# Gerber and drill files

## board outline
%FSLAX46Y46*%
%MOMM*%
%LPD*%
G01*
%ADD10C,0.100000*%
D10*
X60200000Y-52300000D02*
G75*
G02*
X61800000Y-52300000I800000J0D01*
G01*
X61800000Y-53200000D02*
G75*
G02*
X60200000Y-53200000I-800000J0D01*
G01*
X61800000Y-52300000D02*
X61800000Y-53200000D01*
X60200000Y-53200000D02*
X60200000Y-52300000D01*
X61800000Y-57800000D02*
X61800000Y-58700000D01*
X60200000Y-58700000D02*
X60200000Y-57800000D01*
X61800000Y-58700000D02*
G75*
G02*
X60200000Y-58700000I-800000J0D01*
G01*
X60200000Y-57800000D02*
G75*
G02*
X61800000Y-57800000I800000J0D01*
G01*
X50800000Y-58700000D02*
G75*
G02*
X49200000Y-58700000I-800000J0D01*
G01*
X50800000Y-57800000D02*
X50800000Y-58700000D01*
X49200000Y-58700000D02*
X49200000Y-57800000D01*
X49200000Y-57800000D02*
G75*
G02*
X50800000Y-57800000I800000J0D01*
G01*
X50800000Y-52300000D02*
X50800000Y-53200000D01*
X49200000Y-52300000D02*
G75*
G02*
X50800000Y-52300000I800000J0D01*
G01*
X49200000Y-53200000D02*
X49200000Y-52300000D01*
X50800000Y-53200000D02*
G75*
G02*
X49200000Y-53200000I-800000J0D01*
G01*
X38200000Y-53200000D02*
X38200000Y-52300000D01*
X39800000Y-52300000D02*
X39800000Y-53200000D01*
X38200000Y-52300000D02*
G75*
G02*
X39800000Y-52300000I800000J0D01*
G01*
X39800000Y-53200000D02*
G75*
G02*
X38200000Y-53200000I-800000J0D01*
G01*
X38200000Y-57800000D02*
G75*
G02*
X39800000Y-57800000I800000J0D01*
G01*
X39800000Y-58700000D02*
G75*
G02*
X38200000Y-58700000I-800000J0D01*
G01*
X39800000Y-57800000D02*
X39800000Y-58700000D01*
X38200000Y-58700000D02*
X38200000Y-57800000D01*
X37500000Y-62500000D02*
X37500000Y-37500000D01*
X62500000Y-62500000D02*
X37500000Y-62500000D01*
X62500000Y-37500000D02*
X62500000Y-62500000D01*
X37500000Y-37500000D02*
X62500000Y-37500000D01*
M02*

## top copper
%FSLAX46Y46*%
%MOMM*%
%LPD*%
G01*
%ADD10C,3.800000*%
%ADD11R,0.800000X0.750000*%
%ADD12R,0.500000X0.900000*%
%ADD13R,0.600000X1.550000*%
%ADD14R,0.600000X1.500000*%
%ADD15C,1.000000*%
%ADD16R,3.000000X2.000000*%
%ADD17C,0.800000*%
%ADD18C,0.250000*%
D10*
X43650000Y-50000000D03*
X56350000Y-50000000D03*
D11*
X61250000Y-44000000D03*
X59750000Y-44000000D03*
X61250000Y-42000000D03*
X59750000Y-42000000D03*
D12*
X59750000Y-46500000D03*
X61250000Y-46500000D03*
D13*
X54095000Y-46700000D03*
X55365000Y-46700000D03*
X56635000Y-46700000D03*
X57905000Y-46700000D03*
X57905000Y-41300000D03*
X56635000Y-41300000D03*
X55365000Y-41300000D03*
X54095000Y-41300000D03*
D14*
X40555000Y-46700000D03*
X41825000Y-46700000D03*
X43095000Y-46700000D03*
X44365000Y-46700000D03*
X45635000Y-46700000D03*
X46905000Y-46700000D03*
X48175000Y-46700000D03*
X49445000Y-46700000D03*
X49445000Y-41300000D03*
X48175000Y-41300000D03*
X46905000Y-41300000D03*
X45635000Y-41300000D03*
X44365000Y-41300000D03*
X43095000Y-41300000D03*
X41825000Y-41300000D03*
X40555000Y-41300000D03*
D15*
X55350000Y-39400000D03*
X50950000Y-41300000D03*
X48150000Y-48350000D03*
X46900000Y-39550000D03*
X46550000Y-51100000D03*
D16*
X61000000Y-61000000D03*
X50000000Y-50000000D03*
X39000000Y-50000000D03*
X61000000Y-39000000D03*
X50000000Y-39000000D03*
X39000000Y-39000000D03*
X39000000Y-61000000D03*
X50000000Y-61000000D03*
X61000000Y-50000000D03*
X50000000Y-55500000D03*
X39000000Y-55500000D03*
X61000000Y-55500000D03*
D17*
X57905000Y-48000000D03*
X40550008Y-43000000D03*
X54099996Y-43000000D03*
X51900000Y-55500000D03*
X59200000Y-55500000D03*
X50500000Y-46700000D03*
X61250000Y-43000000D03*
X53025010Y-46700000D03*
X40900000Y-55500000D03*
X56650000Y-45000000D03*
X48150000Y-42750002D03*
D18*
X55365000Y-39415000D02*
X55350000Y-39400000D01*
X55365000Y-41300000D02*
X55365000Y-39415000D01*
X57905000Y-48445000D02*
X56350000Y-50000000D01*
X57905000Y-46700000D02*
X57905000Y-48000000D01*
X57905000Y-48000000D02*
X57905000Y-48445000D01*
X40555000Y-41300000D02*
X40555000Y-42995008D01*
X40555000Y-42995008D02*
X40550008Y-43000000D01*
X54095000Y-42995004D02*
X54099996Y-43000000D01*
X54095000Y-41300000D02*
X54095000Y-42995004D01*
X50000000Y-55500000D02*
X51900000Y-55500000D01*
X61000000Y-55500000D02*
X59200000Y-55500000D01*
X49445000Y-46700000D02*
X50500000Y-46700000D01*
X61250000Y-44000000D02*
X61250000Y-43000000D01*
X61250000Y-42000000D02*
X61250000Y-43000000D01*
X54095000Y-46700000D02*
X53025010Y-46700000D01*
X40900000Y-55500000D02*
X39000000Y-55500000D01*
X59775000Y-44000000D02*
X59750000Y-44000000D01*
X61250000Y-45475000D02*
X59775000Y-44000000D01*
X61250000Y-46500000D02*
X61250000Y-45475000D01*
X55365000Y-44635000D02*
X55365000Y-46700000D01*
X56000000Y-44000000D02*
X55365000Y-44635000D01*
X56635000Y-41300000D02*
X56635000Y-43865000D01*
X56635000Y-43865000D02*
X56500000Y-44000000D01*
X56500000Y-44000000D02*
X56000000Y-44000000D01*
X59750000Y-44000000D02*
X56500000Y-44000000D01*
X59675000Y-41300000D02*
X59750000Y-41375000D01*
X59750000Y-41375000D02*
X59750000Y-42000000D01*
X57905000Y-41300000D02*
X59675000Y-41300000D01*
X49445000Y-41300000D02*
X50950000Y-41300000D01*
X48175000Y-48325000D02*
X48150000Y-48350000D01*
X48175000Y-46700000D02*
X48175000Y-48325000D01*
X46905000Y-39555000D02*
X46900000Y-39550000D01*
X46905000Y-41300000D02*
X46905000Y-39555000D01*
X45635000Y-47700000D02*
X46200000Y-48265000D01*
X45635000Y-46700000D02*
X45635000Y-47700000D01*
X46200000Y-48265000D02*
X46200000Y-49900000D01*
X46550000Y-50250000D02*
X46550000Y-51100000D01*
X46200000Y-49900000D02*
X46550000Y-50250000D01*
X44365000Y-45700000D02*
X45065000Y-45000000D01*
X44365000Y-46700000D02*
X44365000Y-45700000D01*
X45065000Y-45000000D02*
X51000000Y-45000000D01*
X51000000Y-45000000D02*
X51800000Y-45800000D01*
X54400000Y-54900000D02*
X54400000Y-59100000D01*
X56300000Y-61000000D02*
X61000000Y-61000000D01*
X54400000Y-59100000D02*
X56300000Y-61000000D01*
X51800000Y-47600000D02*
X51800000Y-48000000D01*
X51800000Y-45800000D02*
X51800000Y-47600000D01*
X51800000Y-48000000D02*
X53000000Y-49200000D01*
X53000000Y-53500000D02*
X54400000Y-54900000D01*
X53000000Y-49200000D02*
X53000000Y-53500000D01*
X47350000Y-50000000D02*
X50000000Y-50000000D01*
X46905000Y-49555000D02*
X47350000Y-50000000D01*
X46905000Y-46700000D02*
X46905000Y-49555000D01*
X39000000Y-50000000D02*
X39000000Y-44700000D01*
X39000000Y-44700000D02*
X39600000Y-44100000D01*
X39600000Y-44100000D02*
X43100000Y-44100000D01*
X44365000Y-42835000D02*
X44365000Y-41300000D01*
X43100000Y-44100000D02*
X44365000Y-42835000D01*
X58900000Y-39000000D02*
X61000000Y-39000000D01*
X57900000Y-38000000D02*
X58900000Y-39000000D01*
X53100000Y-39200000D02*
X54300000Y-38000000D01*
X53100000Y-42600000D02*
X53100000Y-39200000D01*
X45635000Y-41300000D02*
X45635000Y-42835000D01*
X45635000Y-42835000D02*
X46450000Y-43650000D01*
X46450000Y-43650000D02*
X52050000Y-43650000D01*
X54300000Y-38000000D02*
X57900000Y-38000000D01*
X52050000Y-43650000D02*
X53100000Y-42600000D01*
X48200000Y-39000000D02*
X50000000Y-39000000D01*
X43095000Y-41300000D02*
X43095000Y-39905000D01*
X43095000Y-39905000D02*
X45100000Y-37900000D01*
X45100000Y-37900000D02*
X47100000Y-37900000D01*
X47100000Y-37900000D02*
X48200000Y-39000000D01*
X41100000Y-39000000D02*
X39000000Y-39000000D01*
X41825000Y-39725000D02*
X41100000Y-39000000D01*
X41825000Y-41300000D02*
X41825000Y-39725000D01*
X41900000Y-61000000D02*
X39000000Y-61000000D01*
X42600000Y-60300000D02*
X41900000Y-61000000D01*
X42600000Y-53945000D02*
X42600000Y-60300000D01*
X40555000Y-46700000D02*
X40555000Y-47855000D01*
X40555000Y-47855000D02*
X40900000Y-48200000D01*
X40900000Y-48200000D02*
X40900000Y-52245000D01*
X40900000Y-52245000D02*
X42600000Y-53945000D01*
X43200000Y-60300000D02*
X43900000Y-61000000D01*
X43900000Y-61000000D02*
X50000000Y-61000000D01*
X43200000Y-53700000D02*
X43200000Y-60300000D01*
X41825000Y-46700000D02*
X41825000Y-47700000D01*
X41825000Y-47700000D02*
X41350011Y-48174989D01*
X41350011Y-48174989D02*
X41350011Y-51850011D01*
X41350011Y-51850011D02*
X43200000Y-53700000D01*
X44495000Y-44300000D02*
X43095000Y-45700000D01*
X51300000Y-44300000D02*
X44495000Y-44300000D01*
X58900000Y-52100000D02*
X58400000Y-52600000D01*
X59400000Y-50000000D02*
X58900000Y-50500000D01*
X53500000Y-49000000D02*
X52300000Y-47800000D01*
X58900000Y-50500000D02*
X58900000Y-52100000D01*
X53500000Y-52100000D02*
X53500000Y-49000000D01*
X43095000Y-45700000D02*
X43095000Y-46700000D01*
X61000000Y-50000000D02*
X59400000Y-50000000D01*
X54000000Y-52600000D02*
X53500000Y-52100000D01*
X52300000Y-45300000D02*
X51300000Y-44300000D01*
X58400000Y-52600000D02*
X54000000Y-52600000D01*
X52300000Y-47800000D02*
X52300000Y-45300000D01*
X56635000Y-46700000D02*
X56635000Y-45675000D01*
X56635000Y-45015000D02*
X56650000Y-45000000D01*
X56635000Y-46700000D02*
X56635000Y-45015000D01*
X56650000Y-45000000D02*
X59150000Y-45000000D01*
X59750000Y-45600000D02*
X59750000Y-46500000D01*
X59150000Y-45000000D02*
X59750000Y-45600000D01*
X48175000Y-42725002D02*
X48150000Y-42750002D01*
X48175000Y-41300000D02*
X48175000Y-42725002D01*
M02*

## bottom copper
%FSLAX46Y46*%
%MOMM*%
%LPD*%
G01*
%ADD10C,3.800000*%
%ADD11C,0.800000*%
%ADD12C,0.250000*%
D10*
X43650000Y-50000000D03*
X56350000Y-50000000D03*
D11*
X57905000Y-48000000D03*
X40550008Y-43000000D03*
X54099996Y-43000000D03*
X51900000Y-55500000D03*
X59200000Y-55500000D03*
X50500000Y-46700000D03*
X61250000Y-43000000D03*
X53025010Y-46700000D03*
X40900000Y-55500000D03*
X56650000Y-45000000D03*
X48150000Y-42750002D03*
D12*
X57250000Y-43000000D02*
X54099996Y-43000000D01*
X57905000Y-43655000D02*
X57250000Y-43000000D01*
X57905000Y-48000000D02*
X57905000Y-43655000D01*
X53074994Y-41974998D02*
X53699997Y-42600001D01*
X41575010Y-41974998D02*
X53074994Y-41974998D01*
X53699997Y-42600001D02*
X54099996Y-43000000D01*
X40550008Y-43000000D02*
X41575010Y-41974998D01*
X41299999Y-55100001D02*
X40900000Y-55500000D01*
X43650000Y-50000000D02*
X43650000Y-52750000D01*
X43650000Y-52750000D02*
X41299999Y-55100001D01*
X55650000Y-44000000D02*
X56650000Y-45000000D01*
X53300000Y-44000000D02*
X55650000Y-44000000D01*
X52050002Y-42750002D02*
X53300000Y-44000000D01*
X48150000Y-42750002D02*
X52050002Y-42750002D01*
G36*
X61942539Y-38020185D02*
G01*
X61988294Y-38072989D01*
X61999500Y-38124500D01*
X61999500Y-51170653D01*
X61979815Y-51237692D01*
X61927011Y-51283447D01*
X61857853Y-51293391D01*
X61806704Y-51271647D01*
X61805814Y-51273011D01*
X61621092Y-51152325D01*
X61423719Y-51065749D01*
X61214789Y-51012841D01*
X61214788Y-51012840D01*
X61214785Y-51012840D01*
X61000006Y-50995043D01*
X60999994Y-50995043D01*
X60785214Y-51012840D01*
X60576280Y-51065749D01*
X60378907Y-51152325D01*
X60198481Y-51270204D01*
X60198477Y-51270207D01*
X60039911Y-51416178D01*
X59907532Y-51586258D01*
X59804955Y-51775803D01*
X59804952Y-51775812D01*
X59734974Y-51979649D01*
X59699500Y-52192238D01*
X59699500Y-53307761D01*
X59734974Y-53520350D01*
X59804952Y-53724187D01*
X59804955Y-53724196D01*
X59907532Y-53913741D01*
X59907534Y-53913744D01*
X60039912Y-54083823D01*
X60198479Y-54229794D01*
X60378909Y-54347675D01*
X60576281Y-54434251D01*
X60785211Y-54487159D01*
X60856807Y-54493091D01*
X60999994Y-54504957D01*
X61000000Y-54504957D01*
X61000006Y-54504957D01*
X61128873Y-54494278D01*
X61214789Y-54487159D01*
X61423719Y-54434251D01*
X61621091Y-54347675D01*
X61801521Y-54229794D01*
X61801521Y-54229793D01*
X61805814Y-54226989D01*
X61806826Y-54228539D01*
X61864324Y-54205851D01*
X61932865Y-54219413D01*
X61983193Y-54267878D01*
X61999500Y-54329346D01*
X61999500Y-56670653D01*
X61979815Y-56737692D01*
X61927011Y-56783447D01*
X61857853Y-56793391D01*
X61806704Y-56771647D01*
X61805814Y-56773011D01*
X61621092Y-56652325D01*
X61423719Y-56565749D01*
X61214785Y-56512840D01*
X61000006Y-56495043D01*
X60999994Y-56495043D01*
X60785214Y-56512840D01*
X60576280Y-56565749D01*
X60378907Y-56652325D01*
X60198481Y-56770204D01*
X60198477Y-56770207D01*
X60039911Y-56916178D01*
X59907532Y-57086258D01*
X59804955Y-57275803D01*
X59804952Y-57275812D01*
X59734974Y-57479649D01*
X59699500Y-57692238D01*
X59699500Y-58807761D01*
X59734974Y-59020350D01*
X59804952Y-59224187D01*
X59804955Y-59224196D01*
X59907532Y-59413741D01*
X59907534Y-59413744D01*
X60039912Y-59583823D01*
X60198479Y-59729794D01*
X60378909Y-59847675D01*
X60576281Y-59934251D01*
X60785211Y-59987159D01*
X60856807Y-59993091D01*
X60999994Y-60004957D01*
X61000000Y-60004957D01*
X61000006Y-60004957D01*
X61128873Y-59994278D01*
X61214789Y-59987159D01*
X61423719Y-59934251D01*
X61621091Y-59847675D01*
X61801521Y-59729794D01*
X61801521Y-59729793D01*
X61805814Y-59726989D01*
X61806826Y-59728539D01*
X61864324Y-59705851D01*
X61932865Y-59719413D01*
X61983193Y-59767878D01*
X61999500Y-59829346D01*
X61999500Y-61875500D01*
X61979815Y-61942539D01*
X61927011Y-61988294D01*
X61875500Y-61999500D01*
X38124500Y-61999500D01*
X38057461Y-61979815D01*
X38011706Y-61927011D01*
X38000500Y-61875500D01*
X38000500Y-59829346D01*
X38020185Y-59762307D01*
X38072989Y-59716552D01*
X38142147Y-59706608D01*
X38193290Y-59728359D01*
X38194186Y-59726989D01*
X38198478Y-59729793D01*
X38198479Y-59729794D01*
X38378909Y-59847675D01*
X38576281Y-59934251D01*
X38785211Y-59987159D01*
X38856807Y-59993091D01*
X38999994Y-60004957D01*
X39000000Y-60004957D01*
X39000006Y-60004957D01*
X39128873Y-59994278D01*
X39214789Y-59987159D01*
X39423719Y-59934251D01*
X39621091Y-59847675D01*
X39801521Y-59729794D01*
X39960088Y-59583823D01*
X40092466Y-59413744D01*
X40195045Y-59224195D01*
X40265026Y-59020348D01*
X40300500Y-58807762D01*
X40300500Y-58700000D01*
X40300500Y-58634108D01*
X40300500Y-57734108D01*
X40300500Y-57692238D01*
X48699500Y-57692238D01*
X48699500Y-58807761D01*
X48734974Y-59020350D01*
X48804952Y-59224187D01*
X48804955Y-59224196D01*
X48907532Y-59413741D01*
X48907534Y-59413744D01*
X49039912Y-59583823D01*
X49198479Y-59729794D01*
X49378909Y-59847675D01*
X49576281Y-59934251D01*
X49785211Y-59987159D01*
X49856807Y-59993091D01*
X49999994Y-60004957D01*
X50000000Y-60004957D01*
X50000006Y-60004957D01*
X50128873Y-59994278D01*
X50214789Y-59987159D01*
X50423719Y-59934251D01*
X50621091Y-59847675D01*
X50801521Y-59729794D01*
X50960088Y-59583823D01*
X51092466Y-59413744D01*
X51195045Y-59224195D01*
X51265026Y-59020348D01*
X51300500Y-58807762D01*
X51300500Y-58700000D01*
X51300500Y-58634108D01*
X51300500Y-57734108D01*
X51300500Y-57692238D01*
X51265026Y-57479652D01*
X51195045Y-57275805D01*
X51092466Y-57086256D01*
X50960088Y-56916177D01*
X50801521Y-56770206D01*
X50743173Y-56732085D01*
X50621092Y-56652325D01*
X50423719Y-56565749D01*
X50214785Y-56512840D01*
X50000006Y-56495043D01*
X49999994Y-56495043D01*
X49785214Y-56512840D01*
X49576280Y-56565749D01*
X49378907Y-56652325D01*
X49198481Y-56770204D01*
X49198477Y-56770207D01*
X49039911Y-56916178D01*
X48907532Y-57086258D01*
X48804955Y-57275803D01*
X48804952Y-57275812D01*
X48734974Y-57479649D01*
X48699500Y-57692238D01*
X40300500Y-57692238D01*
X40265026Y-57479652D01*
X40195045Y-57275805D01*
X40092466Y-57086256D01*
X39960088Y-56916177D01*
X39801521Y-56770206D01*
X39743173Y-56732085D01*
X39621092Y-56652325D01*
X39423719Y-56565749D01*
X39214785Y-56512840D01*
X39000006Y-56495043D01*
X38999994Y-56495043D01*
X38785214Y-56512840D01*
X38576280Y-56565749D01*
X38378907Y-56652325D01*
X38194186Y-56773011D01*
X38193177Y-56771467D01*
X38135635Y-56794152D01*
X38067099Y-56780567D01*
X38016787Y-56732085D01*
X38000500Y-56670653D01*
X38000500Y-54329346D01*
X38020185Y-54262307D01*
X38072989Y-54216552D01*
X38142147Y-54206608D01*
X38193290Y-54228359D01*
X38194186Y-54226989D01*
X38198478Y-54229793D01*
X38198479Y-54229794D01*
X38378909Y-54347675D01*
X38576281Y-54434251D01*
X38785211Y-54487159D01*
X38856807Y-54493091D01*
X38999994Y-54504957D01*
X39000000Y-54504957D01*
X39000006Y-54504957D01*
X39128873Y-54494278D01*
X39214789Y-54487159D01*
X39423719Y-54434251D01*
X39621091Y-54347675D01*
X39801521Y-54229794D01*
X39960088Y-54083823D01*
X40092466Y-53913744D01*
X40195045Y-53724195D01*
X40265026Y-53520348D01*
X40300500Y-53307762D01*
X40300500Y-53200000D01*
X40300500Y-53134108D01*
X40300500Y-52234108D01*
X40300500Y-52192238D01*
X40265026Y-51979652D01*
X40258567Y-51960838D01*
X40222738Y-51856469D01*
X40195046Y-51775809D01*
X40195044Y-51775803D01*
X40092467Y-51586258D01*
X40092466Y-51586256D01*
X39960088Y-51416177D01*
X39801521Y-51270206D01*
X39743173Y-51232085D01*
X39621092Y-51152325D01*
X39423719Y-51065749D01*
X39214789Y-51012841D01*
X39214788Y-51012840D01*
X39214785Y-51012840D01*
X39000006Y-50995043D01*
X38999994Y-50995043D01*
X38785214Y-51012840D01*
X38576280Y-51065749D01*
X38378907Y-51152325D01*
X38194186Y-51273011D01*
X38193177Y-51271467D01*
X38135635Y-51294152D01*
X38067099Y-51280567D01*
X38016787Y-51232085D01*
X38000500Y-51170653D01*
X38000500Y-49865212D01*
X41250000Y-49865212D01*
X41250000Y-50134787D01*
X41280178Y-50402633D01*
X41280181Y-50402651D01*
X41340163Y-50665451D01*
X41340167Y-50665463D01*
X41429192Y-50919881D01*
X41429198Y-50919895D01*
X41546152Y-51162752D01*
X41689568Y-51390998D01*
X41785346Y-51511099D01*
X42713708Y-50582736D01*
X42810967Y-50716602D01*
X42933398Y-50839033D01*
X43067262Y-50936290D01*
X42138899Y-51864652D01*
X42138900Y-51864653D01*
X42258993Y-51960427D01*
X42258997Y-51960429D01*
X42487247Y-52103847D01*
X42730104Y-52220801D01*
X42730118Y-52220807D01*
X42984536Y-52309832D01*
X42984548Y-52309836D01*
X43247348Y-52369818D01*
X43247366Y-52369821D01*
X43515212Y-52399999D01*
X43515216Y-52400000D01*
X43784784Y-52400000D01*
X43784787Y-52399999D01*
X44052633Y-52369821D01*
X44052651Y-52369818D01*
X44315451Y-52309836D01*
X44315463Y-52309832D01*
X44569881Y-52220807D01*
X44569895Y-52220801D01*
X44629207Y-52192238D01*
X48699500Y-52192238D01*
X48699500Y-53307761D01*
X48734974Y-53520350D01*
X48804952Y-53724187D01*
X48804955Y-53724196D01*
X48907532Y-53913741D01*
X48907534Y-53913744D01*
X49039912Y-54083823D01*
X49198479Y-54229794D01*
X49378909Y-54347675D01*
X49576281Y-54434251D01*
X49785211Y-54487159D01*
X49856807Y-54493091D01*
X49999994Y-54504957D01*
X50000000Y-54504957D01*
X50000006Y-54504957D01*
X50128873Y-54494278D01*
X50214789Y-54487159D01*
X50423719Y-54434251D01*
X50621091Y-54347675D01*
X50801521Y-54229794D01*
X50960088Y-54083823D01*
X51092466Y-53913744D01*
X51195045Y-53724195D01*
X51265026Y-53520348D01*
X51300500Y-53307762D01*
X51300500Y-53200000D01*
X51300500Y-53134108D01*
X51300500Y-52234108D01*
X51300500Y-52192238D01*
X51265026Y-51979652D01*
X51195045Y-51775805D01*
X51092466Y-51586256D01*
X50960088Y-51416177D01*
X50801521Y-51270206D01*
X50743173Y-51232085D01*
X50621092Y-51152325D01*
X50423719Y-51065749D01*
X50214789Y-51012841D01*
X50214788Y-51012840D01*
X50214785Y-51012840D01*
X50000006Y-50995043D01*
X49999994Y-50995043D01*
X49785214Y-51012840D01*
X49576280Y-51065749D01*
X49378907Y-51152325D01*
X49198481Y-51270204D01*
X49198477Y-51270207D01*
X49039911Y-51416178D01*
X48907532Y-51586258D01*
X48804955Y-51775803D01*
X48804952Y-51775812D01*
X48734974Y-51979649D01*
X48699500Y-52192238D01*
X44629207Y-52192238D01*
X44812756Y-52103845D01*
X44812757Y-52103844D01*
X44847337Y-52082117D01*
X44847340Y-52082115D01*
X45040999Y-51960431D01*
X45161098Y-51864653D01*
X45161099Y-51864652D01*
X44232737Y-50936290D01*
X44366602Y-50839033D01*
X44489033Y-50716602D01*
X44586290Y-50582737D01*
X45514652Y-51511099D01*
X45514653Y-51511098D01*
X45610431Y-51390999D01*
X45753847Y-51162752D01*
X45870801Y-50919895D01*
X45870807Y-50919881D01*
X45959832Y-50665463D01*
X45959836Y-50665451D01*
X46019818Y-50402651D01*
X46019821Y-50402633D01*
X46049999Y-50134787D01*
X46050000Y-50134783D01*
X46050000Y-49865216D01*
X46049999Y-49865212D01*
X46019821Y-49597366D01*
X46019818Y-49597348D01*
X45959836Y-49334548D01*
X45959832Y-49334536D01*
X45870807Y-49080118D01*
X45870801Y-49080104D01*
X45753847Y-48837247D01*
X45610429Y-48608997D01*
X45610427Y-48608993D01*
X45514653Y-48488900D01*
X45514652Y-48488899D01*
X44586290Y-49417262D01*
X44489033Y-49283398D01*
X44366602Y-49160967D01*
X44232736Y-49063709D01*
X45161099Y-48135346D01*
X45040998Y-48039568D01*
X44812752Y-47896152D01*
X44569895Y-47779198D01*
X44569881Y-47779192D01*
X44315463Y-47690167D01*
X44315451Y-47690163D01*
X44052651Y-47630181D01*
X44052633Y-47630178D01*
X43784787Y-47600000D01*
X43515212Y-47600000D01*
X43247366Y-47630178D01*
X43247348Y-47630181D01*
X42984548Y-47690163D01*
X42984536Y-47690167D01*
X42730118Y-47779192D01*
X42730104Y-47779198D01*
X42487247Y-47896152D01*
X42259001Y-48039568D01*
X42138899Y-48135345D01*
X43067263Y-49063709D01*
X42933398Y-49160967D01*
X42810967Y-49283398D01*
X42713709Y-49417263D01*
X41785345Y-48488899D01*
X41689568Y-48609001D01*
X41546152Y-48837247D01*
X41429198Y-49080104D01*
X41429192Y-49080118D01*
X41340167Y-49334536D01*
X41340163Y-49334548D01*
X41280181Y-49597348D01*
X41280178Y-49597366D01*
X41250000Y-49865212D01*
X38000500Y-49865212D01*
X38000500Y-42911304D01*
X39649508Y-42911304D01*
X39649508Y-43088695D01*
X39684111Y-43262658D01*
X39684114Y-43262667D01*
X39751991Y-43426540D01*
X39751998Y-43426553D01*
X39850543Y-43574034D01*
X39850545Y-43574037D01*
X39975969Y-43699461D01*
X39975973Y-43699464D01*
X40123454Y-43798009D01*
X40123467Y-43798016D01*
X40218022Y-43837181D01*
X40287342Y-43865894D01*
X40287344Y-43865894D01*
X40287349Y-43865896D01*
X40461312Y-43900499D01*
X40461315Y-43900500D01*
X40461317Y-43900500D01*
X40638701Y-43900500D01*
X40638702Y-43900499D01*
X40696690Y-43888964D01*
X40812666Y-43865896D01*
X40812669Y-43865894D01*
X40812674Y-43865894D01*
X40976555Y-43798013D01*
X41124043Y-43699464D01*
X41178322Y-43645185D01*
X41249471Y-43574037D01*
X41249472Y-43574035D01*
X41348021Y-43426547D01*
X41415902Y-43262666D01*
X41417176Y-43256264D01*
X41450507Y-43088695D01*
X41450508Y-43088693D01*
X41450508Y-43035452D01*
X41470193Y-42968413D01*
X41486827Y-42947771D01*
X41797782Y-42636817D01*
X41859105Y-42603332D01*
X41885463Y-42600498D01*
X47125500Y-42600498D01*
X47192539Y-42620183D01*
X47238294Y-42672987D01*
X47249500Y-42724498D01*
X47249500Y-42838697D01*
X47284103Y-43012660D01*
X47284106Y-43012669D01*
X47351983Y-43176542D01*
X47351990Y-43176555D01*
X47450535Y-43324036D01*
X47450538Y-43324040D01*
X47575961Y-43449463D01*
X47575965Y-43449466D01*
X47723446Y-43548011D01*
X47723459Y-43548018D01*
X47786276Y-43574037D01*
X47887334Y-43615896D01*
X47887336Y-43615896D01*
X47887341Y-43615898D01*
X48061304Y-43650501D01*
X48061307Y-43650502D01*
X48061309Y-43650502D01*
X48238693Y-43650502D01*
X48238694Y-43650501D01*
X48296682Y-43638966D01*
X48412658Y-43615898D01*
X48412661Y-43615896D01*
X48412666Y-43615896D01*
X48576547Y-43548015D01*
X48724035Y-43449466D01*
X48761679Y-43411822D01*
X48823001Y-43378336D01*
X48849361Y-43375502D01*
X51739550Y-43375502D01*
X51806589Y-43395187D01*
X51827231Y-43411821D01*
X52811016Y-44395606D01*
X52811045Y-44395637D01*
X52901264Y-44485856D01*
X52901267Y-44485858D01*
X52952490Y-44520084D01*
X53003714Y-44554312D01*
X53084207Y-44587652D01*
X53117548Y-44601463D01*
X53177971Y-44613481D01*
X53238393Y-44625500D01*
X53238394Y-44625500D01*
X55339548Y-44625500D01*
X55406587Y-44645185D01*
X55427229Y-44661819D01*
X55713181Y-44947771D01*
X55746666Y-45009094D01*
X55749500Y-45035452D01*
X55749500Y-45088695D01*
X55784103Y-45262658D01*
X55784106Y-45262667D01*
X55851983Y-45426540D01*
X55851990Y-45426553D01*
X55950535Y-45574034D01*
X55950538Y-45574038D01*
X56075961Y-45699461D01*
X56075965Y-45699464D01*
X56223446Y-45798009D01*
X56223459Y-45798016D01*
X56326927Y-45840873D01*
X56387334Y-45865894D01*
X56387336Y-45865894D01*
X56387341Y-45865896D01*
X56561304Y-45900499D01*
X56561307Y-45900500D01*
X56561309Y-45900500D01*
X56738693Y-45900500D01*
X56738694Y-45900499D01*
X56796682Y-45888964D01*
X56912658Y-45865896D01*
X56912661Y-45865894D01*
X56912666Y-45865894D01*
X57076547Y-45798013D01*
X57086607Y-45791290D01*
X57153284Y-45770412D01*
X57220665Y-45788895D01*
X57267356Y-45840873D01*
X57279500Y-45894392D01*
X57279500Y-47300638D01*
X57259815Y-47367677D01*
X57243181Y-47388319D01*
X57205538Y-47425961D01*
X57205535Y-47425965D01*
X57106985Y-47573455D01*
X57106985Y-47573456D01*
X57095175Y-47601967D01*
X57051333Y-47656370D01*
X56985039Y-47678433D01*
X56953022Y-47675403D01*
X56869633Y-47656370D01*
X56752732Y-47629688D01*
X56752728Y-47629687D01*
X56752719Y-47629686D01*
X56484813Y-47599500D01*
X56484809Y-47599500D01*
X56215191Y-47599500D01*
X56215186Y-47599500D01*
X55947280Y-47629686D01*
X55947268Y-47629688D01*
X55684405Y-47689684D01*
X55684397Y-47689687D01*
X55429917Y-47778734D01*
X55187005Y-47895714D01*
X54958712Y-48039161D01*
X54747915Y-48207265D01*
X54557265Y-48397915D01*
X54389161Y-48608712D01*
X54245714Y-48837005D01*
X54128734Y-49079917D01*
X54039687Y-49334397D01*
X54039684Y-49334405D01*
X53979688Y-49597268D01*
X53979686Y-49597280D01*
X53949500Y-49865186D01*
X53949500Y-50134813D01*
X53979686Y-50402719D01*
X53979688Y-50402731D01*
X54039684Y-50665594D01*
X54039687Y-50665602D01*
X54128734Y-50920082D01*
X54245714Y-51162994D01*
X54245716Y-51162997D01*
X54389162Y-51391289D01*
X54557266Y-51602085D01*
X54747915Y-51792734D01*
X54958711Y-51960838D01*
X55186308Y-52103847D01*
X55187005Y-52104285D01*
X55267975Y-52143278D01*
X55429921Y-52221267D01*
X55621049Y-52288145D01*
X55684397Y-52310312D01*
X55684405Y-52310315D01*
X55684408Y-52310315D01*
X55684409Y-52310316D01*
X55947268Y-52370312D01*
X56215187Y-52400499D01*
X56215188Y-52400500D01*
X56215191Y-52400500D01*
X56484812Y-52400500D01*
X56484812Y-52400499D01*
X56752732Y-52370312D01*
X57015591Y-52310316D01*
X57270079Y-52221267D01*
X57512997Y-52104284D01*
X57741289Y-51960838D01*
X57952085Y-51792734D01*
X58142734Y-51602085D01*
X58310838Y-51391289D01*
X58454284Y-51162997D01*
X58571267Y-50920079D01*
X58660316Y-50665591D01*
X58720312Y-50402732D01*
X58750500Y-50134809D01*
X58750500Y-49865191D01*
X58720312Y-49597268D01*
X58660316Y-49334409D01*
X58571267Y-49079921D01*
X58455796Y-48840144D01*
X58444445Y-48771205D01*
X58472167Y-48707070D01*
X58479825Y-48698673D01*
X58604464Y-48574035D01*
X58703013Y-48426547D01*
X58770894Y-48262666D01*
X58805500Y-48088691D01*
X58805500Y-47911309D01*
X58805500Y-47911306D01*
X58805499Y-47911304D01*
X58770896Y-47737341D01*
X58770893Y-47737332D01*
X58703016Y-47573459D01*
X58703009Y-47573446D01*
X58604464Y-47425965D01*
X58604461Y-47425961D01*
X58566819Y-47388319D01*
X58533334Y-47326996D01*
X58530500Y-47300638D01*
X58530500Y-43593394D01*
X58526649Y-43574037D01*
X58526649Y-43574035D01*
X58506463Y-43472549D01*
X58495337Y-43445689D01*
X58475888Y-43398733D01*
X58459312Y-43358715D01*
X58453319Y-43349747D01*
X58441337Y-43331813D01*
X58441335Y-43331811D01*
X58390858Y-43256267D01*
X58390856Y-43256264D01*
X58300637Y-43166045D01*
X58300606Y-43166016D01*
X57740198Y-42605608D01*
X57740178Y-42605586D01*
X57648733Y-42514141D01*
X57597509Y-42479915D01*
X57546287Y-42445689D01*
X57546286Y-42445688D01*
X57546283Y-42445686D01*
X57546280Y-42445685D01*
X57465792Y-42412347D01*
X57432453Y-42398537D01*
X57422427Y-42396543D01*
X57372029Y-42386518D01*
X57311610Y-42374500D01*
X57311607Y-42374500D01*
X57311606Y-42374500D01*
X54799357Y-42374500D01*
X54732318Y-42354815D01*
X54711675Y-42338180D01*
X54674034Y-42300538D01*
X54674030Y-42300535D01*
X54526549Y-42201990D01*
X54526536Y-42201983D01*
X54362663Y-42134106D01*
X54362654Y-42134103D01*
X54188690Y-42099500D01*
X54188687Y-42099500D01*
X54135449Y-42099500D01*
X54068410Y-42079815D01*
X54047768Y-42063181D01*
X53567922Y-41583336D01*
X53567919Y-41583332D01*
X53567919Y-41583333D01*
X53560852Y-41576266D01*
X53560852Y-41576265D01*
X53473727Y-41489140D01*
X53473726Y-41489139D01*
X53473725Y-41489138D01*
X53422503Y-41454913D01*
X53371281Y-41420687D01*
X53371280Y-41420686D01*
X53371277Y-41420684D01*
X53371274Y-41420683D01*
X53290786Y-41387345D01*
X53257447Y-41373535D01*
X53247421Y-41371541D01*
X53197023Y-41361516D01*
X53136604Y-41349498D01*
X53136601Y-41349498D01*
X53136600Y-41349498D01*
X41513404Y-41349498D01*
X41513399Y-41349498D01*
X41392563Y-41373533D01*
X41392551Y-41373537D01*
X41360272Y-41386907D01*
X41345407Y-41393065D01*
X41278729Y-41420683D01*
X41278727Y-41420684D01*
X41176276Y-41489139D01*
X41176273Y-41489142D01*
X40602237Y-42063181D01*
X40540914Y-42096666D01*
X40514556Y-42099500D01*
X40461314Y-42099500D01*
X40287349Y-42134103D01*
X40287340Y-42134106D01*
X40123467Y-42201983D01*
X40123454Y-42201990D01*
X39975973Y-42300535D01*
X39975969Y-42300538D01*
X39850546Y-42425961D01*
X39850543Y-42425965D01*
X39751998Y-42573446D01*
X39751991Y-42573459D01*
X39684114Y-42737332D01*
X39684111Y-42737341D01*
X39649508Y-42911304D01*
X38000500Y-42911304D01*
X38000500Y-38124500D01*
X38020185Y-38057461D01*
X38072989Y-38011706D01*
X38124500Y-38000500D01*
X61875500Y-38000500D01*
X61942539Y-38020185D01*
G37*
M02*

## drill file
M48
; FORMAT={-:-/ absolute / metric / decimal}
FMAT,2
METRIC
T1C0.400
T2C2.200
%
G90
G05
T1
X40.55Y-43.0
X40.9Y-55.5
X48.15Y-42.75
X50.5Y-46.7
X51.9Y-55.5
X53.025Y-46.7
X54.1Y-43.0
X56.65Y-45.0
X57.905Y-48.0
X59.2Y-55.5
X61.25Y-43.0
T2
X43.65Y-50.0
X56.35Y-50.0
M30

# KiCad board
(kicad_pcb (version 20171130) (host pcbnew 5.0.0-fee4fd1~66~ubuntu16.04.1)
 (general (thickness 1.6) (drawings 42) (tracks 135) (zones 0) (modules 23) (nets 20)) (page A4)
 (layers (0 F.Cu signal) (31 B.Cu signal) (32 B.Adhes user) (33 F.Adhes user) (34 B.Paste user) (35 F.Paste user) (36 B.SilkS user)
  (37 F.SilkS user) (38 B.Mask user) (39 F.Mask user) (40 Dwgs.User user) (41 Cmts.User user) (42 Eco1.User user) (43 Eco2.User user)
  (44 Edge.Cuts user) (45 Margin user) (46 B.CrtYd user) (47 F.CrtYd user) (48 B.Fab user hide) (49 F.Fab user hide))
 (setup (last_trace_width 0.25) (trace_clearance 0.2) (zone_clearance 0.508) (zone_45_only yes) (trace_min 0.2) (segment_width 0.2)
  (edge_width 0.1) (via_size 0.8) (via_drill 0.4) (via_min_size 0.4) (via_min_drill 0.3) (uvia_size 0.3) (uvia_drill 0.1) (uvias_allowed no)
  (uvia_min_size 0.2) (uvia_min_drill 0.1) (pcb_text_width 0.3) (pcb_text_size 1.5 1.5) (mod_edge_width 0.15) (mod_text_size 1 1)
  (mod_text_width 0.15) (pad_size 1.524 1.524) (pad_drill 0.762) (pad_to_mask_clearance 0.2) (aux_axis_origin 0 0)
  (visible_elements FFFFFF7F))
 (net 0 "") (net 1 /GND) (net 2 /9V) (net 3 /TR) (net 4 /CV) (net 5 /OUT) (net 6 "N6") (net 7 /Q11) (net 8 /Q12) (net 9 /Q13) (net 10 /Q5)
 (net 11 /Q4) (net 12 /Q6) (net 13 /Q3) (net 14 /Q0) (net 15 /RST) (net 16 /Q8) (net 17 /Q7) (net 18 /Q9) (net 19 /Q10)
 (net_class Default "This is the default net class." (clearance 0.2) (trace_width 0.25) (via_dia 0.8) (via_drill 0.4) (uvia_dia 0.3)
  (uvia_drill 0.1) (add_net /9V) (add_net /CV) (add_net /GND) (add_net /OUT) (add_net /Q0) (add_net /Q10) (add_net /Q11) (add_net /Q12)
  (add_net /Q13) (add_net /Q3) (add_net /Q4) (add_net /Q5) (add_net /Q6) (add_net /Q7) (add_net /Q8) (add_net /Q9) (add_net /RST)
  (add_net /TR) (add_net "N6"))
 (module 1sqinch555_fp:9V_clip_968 (layer F.Cu) (at 50 50)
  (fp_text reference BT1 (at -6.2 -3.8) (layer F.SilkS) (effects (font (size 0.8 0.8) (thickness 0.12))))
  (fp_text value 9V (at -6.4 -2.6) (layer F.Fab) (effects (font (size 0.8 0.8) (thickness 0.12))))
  (pad 2 thru_hole circle (at -6.35 0) (size 3.8 3.8) (drill 2.2) (layers *.Cu *.Mask F.SilkS) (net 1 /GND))
  (pad 1 thru_hole circle (at 6.35 0) (size 3.8 3.8) (drill 2.2) (layers *.Cu *.Mask F.SilkS) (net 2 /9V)))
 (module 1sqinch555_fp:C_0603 (layer F.Cu) (at 60.5 44)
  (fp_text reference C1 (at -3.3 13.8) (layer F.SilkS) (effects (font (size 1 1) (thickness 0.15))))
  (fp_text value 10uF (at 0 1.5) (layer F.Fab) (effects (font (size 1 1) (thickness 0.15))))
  (pad 2 smd rect (at 0.75 0) (size 0.8 0.75) (layers F.Cu F.Paste F.Mask) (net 1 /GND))
  (pad 1 smd rect (at -0.75 0) (size 0.8 0.75) (layers F.Cu F.Paste F.Mask) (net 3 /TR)))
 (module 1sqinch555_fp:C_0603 (layer F.Cu) (at 60.5 42)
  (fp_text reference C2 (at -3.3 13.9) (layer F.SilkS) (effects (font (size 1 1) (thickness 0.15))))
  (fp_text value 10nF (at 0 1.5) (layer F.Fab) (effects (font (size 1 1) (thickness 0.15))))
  (pad 2 smd rect (at 0.75 0) (size 0.8 0.75) (layers F.Cu F.Paste F.Mask) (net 1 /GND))
  (pad 1 smd rect (at -0.75 0) (size 0.8 0.75) (layers F.Cu F.Paste F.Mask) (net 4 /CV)))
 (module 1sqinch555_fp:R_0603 (layer F.Cu) (at 60.5 46.5)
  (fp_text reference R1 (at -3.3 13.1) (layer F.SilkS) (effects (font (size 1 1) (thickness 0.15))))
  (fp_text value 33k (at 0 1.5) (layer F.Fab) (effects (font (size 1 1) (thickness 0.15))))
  (pad 1 smd rect (at -0.75 0) (size 0.5 0.9) (layers F.Cu F.Paste F.Mask) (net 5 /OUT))
  (pad 2 smd rect (at 0.75 0) (size 0.5 0.9) (layers F.Cu F.Paste F.Mask) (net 3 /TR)))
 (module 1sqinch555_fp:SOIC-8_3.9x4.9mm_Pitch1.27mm (layer F.Cu) (at 56 44 90)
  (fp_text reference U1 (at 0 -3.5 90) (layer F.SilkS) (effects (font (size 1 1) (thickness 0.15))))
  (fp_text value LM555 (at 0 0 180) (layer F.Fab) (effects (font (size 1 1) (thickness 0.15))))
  (pad 1 smd rect (at -2.7 -1.905 90) (size 1.55 0.6) (layers F.Cu F.Paste F.Mask) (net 1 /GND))
  (pad 2 smd rect (at -2.7 -0.635 90) (size 1.55 0.6) (layers F.Cu F.Paste F.Mask) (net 3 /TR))
  (pad 3 smd rect (at -2.7 0.635 90) (size 1.55 0.6) (layers F.Cu F.Paste F.Mask) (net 5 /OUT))
  (pad 4 smd rect (at -2.7 1.905 90) (size 1.55 0.6) (layers F.Cu F.Paste F.Mask) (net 2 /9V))
  (pad 5 smd rect (at 2.7 1.905 90) (size 1.55 0.6) (layers F.Cu F.Paste F.Mask) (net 4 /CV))
  (pad 6 smd rect (at 2.7 0.635 90) (size 1.55 0.6) (layers F.Cu F.Paste F.Mask) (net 3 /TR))
  (pad 7 smd rect (at 2.7 -0.635 90) (size 1.55 0.6) (layers F.Cu F.Paste F.Mask) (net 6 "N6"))
  (pad 8 smd rect (at 2.7 -1.905 90) (size 1.55 0.6) (layers F.Cu F.Paste F.Mask) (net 2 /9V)))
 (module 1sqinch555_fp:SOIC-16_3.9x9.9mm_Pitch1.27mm (layer F.Cu) (at 45 44 90)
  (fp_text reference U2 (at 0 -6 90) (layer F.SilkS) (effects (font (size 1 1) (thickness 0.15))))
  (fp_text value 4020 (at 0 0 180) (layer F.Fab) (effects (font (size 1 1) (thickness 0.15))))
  (pad 1 smd rect (at -2.7 -4.445 90) (size 1.5 0.6) (layers F.Cu F.Paste F.Mask) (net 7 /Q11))
  (pad 2 smd rect (at -2.7 -3.175 90) (size 1.5 0.6) (layers F.Cu F.Paste F.Mask) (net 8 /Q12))
  (pad 3 smd rect (at -2.7 -1.905 90) (size 1.5 0.6) (layers F.Cu F.Paste F.Mask) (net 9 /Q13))
  (pad 4 smd rect (at -2.7 -0.635 90) (size 1.5 0.6) (layers F.Cu F.Paste F.Mask) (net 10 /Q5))
  (pad 5 smd rect (at -2.7 0.635 90) (size 1.5 0.6) (layers F.Cu F.Paste F.Mask) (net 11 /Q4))
  (pad 6 smd rect (at -2.7 1.905 90) (size 1.5 0.6) (layers F.Cu F.Paste F.Mask) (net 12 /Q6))
  (pad 7 smd rect (at -2.7 3.175 90) (size 1.5 0.6) (layers F.Cu F.Paste F.Mask) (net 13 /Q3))
  (pad 8 smd rect (at -2.7 4.445 90) (size 1.5 0.6) (layers F.Cu F.Paste F.Mask) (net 1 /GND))
  (pad 9 smd rect (at 2.7 4.445 90) (size 1.5 0.6) (layers F.Cu F.Paste F.Mask) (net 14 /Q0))
  (pad 10 smd rect (at 2.7 3.175 90) (size 1.5 0.6) (layers F.Cu F.Paste F.Mask) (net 5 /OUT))
  (pad 11 smd rect (at 2.7 1.905 90) (size 1.5 0.6) (layers F.Cu F.Paste F.Mask) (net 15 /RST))
  (pad 12 smd rect (at 2.7 0.635 90) (size 1.5 0.6) (layers F.Cu F.Paste F.Mask) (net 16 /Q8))
  (pad 13 smd rect (at 2.7 -0.635 90) (size 1.5 0.6) (layers F.Cu F.Paste F.Mask) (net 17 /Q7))
  (pad 14 smd rect (at 2.7 -1.905 90) (size 1.5 0.6) (layers F.Cu F.Paste F.Mask) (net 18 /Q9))
  (pad 15 smd rect (at 2.7 -3.175 90) (size 1.5 0.6) (layers F.Cu F.Paste F.Mask) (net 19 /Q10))
  (pad 16 smd rect (at 2.7 -4.445 90) (size 1.5 0.6) (layers F.Cu F.Paste F.Mask) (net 2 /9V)))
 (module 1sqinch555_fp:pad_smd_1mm (layer F.Cu) (at 55.35 39.4)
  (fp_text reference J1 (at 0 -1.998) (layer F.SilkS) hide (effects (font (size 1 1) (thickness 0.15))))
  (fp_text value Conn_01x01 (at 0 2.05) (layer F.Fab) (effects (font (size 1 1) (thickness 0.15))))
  (pad 1 smd circle (at 0 0) (size 1 1) (layers F.Cu F.Mask) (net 6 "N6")))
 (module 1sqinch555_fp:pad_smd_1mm (layer F.Cu) (at 50.95 41.3)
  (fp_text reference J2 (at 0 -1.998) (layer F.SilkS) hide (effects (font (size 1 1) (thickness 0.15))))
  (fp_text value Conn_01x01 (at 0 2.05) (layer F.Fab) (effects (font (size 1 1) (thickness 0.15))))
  (pad 1 smd circle (at 0 0) (size 1 1) (layers F.Cu F.Mask) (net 14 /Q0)))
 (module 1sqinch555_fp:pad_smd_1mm (layer F.Cu) (at 48.15 48.35)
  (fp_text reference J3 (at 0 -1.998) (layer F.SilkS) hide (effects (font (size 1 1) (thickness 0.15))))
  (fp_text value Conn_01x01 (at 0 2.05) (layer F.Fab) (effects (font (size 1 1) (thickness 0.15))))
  (pad 1 smd circle (at 0 0) (size 1 1) (layers F.Cu F.Mask) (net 13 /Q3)))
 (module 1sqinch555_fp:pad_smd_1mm (layer F.Cu) (at 46.9 39.55)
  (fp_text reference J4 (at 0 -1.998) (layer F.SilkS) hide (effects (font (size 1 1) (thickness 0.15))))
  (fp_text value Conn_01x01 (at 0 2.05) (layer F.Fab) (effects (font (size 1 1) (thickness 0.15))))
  (pad 1 smd circle (at 0 0) (size 1 1) (layers F.Cu F.Mask) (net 15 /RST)))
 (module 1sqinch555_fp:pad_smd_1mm (layer F.Cu) (at 46.55 51.1)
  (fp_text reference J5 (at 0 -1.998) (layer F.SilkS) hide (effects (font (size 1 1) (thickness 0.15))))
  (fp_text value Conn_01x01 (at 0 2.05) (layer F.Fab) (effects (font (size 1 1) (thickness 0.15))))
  (pad 1 smd circle (at 0 0) (size 1 1) (layers F.Cu F.Mask) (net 11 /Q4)))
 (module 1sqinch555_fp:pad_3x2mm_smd (layer F.Cu) (at 61 61)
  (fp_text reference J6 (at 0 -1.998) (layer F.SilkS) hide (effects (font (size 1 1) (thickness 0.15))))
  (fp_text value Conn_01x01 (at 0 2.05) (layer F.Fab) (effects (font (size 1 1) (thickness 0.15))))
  (pad 1 smd rect (at 0 0) (size 3 2) (layers F.Cu F.Mask) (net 10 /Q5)))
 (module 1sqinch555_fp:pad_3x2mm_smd (layer F.Cu) (at 50 50)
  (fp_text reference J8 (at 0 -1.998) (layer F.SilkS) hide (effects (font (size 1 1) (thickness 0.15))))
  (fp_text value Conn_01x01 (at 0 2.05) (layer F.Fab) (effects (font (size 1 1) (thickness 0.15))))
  (pad 1 smd rect (at 0 0) (size 3 2) (layers F.Cu F.Mask) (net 12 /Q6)))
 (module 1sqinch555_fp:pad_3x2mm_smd (layer F.Cu) (at 39 50)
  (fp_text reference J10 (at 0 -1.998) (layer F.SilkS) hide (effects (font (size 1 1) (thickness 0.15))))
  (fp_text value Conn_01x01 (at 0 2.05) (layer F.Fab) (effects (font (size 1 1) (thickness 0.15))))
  (pad 1 smd rect (at 0 0) (size 3 2) (layers F.Cu F.Mask) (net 17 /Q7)))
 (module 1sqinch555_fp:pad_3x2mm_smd (layer F.Cu) (at 61 39)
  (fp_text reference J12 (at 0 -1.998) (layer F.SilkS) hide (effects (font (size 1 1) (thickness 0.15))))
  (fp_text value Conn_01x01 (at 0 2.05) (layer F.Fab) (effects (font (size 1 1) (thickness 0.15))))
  (pad 1 smd rect (at 0 0) (size 3 2) (layers F.Cu F.Mask) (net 16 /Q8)))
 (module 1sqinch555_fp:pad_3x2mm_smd (layer F.Cu) (at 50 39)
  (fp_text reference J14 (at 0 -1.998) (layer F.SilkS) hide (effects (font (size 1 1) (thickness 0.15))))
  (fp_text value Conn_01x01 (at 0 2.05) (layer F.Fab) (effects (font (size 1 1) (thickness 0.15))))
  (pad 1 smd rect (at 0 0) (size 3 2) (layers F.Cu F.Mask) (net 18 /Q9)))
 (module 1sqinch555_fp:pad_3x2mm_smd (layer F.Cu) (at 39 39)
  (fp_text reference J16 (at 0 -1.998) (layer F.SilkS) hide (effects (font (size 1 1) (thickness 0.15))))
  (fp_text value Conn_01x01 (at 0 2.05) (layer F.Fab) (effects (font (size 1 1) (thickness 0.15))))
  (pad 1 smd rect (at 0 0) (size 3 2) (layers F.Cu F.Mask) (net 19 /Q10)))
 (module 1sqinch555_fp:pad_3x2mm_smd (layer F.Cu) (at 39 61)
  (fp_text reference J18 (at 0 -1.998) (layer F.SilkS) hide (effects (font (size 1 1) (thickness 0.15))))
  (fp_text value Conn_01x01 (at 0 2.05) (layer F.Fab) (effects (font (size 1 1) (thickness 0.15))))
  (pad 1 smd rect (at 0 0) (size 3 2) (layers F.Cu F.Mask) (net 7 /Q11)))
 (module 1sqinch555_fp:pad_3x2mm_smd (layer F.Cu) (at 50 61)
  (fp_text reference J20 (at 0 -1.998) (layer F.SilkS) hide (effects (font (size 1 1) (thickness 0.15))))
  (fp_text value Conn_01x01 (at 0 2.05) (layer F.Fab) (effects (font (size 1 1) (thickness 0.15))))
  (pad 1 smd rect (at 0 0) (size 3 2) (layers F.Cu F.Mask) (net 8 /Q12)))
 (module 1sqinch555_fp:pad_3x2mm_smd (layer F.Cu) (at 61 50)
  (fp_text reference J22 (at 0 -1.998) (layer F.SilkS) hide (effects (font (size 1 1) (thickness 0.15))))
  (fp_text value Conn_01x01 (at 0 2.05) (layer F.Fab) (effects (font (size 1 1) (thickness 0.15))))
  (pad 1 smd rect (at 0 0) (size 3 2) (layers F.Cu F.Mask) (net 9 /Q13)))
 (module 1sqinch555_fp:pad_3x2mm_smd (layer F.Cu) (at 50 55.5)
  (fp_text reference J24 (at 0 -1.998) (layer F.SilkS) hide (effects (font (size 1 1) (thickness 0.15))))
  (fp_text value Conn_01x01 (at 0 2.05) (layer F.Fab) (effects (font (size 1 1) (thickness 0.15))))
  (pad 1 smd rect (at 0 0) (size 3 2) (layers F.Cu F.Mask) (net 1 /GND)))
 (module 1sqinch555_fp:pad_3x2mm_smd (layer F.Cu) (at 39 55.5)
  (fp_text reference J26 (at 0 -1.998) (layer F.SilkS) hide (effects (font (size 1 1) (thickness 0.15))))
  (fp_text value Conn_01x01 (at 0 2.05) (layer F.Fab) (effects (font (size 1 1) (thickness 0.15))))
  (pad 1 smd rect (at 0 0) (size 3 2) (layers F.Cu F.Mask) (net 1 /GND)))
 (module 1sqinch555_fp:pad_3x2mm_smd (layer F.Cu) (at 61 55.5)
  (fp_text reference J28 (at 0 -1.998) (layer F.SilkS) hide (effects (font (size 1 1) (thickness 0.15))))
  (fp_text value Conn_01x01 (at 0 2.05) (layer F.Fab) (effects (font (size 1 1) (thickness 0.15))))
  (pad 1 smd rect (at 0 0) (size 3 2) (layers F.Cu F.Mask) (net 1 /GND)))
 (gr_arc (start 61 52.3) (end 61.8 52.3) (angle -180) (layer Edge.Cuts) (width 0.1))
 (gr_arc (start 61 53.2) (end 60.2 53.2) (angle -180) (layer Edge.Cuts) (width 0.1))
 (gr_line (start 61.8 52.3) (end 61.8 53.2) (layer Edge.Cuts) (width 0.1))
 (gr_line (start 60.2 53.2) (end 60.2 52.3) (layer Edge.Cuts) (width 0.1))
 (gr_line (start 61.8 57.8) (end 61.8 58.7) (layer Edge.Cuts) (width 0.1))
 (gr_line (start 60.2 58.7) (end 60.2 57.8) (layer Edge.Cuts) (width 0.1))
 (gr_arc (start 61 58.7) (end 60.2 58.7) (angle -180) (layer Edge.Cuts) (width 0.1))
 (gr_arc (start 61 57.8) (end 61.8 57.8) (angle -180) (layer Edge.Cuts) (width 0.1))
 (gr_arc (start 50 58.7) (end 49.2 58.7) (angle -180) (layer Edge.Cuts) (width 0.1))
 (gr_line (start 50.8 57.8) (end 50.8 58.7) (layer Edge.Cuts) (width 0.1))
 (gr_line (start 49.2 58.7) (end 49.2 57.8) (layer Edge.Cuts) (width 0.1))
 (gr_arc (start 50 57.8) (end 50.8 57.8) (angle -180) (layer Edge.Cuts) (width 0.1))
 (gr_line (start 50.8 52.3) (end 50.8 53.2) (layer Edge.Cuts) (width 0.1))
 (gr_arc (start 50 52.3) (end 50.8 52.3) (angle -180) (layer Edge.Cuts) (width 0.1))
 (gr_line (start 49.2 53.2) (end 49.2 52.3) (layer Edge.Cuts) (width 0.1))
 (gr_arc (start 50 53.2) (end 49.2 53.2) (angle -180) (layer Edge.Cuts) (width 0.1))
 (gr_line (start 38.2 53.2) (end 38.2 52.3) (layer Edge.Cuts) (width 0.1))
 (gr_line (start 39.8 52.3) (end 39.8 53.2) (layer Edge.Cuts) (width 0.1))
 (gr_arc (start 39 52.3) (end 39.8 52.3) (angle -180) (layer Edge.Cuts) (width 0.1))
 (gr_arc (start 39 53.2) (end 38.2 53.2) (angle -180) (layer Edge.Cuts) (width 0.1))
 (gr_arc (start 39 57.8) (end 39.8 57.8) (angle -180) (layer Edge.Cuts) (width 0.1))
 (gr_arc (start 39 58.7) (end 38.2 58.7) (angle -180) (layer Edge.Cuts) (width 0.1))
 (gr_line (start 39.8 57.8) (end 39.8 58.7) (layer Edge.Cuts) (width 0.1))
 (gr_line (start 38.2 58.7) (end 38.2 57.8) (layer Edge.Cuts) (width 0.1))
 (gr_line (start 37.5 62.5) (end 37.5 37.5) (layer Edge.Cuts) (width 0.1))
 (gr_line (start 62.5 62.5) (end 37.5 62.5) (layer Edge.Cuts) (width 0.1))
 (gr_line (start 62.5 37.5) (end 62.5 62.5) (layer Edge.Cuts) (width 0.1))
 (gr_line (start 37.5 37.5) (end 62.5 37.5) (layer Edge.Cuts) (width 0.1))
 (segment (start 55.365 39.415) (end 55.35 39.4) (width 0.25) (layer F.Cu) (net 6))
 (segment (start 55.365 41.3) (end 55.365 39.415) (width 0.25) (layer F.Cu) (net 6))
 (segment (start 57.905 48.445) (end 56.35 50) (width 0.25) (layer F.Cu) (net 2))
 (via (at 57.905 48) (size 0.8) (drill 0.4) (layers F.Cu B.Cu) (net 2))
 (segment (start 57.905 46.7) (end 57.905 48) (width 0.25) (layer F.Cu) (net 2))
 (segment (start 57.905 48) (end 57.905 48.445) (width 0.25) (layer F.Cu) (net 2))
 (via (at 40.550008 43) (size 0.8) (drill 0.4) (layers F.Cu B.Cu) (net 2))
 (segment (start 40.555 41.3) (end 40.555 42.995008) (width 0.25) (layer F.Cu) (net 2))
 (segment (start 40.555 42.995008) (end 40.550008 43) (width 0.25) (layer F.Cu) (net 2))
 (segment (start 54.095 42.995004) (end 54.099996 43) (width 0.25) (layer F.Cu) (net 2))
 (segment (start 54.095 41.3) (end 54.095 42.995004) (width 0.25) (layer F.Cu) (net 2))
 (via (at 54.099996 43) (size 0.8) (drill 0.4) (layers F.Cu B.Cu) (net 2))
 (segment (start 57.25 43) (end 54.099996 43) (width 0.25) (layer B.Cu) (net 2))
 (segment (start 57.905 43.655) (end 57.25 43) (width 0.25) (layer B.Cu) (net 2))
 (segment (start 57.905 48) (end 57.905 43.655) (width 0.25) (layer B.Cu) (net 2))
 (segment (start 53.074994 41.974998) (end 53.699997 42.600001) (width 0.25) (layer B.Cu) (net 2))
 (segment (start 41.57501 41.974998) (end 53.074994 41.974998) (width 0.25) (layer B.Cu) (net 2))
 (segment (start 53.699997 42.600001) (end 54.099996 43) (width 0.25) (layer B.Cu) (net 2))
 (segment (start 40.550008 43) (end 41.57501 41.974998) (width 0.25) (layer B.Cu) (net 2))
 (via (at 51.9 55.5) (size 0.8) (drill 0.4) (layers F.Cu B.Cu) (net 1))
 (segment (start 50 55.5) (end 51.9 55.5) (width 0.25) (layer F.Cu) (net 1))
 (via (at 59.2 55.5) (size 0.8) (drill 0.4) (layers F.Cu B.Cu) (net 1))
 (segment (start 61 55.5) (end 59.2 55.5) (width 0.25) (layer F.Cu) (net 1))
 (via (at 50.5 46.7) (size 0.8) (drill 0.4) (layers F.Cu B.Cu) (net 1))
 (segment (start 49.445 46.7) (end 50.5 46.7) (width 0.25) (layer F.Cu) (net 1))
 (via (at 61.25 43) (size 0.8) (drill 0.4) (layers F.Cu B.Cu) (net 1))
 (segment (start 61.25 44) (end 61.25 43) (width 0.25) (layer F.Cu) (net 1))
 (segment (start 61.25 42) (end 61.25 43) (width 0.25) (layer F.Cu) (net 1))
 (via (at 53.02501 46.7) (size 0.8) (drill 0.4) (layers F.Cu B.Cu) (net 1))
 (segment (start 54.095 46.7) (end 53.02501 46.7) (width 0.25) (layer F.Cu) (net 1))
 (via (at 40.9 55.5) (size 0.8) (drill 0.4) (layers F.Cu B.Cu) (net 1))
 (segment (start 41.299999 55.100001) (end 40.9 55.5) (width 0.25) (layer B.Cu) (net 1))
 (segment (start 43.65 50) (end 43.65 52.75) (width 0.25) (layer B.Cu) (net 1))
 (segment (start 43.65 52.75) (end 41.299999 55.100001) (width 0.25) (layer B.Cu) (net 1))
 (segment (start 40.9 55.5) (end 39 55.5) (width 0.25) (layer F.Cu) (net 1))
 (segment (start 59.775 44) (end 59.75 44) (width 0.25) (layer F.Cu) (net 3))
 (segment (start 61.25 45.475) (end 59.775 44) (width 0.25) (layer F.Cu) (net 3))
 (segment (start 61.25 46.5) (end 61.25 45.475) (width 0.25) (layer F.Cu) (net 3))
 (segment (start 55.365 44.635) (end 55.365 46.7) (width 0.25) (layer F.Cu) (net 3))
 (segment (start 56 44) (end 55.365 44.635) (width 0.25) (layer F.Cu) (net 3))
 (segment (start 56.635 41.3) (end 56.635 43.865) (width 0.25) (layer F.Cu) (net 3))
 (segment (start 56.635 43.865) (end 56.5 44) (width 0.25) (layer F.Cu) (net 3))
 (segment (start 56.5 44) (end 56 44) (width 0.25) (layer F.Cu) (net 3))
 (segment (start 59.75 44) (end 56.5 44) (width 0.25) (layer F.Cu) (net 3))
 (segment (start 59.675 41.3) (end 59.75 41.375) (width 0.25) (layer F.Cu) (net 4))
 (segment (start 59.75 41.375) (end 59.75 42) (width 0.25) (layer F.Cu) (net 4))
 (segment (start 57.905 41.3) (end 59.675 41.3) (width 0.25) (layer F.Cu) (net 4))
 (segment (start 49.445 41.3) (end 50.95 41.3) (width 0.25) (layer F.Cu) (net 14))
 (segment (start 48.175 48.325) (end 48.15 48.35) (width 0.25) (layer F.Cu) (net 13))
 (segment (start 48.175 46.7) (end 48.175 48.325) (width 0.25) (layer F.Cu) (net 13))
 (segment (start 46.905 39.555) (end 46.9 39.55) (width 0.25) (layer F.Cu) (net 15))
 (segment (start 46.905 41.3) (end 46.905 39.555) (width 0.25) (layer F.Cu) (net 15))
 (segment (start 45.635 47.7) (end 46.2 48.265) (width 0.25) (layer F.Cu) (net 11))
 (segment (start 45.635 46.7) (end 45.635 47.7) (width 0.25) (layer F.Cu) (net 11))
 (segment (start 46.2 48.265) (end 46.2 49.9) (width 0.25) (layer F.Cu) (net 11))
 (segment (start 46.55 50.25) (end 46.55 51.1) (width 0.25) (layer F.Cu) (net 11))
 (segment (start 46.2 49.9) (end 46.55 50.25) (width 0.25) (layer F.Cu) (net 11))
 (segment (start 44.365 45.7) (end 45.065 45) (width 0.25) (layer F.Cu) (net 10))
 (segment (start 44.365 46.7) (end 44.365 45.7) (width 0.25) (layer F.Cu) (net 10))
 (segment (start 45.065 45) (end 51 45) (width 0.25) (layer F.Cu) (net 10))
 (segment (start 51 45) (end 51.8 45.8) (width 0.25) (layer F.Cu) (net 10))
 (segment (start 54.4 54.9) (end 54.4 59.1) (width 0.25) (layer F.Cu) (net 10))
 (segment (start 56.3 61) (end 61 61) (width 0.25) (layer F.Cu) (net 10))
 (segment (start 54.4 59.1) (end 56.3 61) (width 0.25) (layer F.Cu) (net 10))
 (segment (start 51.8 47.6) (end 51.8 48) (width 0.25) (layer F.Cu) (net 10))
 (segment (start 51.8 45.8) (end 51.8 47.6) (width 0.25) (layer F.Cu) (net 10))
 (segment (start 51.8 48) (end 53 49.2) (width 0.25) (layer F.Cu) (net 10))
 (segment (start 53 53.5) (end 54.4 54.9) (width 0.25) (layer F.Cu) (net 10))
 (segment (start 53 49.2) (end 53 53.5) (width 0.25) (layer F.Cu) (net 10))
 (segment (start 47.35 50) (end 50 50) (width 0.25) (layer F.Cu) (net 12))
 (segment (start 46.905 49.555) (end 47.35 50) (width 0.25) (layer F.Cu) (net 12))
 (segment (start 46.905 46.7) (end 46.905 49.555) (width 0.25) (layer F.Cu) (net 12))
 (segment (start 39 50) (end 39 44.7) (width 0.25) (layer F.Cu) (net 17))
 (segment (start 39 44.7) (end 39.6 44.1) (width 0.25) (layer F.Cu) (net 17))
 (segment (start 39.6 44.1) (end 43.1 44.1) (width 0.25) (layer F.Cu) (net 17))
 (segment (start 44.365 42.835) (end 44.365 41.3) (width 0.25) (layer F.Cu) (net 17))
 (segment (start 43.1 44.1) (end 44.365 42.835) (width 0.25) (layer F.Cu) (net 17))
 (segment (start 58.9 39) (end 61 39) (width 0.25) (layer F.Cu) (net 16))
 (segment (start 57.9 38) (end 58.9 39) (width 0.25) (layer F.Cu) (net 16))
 (segment (start 53.1 39.2) (end 54.3 38) (width 0.25) (layer F.Cu) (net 16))
 (segment (start 53.1 42.6) (end 53.1 39.2) (width 0.25) (layer F.Cu) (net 16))
 (segment (start 45.635 41.3) (end 45.635 42.835) (width 0.25) (layer F.Cu) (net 16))
 (segment (start 45.635 42.835) (end 46.45 43.65) (width 0.25) (layer F.Cu) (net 16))
 (segment (start 46.45 43.65) (end 52.05 43.65) (width 0.25) (layer F.Cu) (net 16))
 (segment (start 54.3 38) (end 57.9 38) (width 0.25) (layer F.Cu) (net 16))
 (segment (start 52.05 43.65) (end 53.1 42.6) (width 0.25) (layer F.Cu) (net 16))
 (segment (start 48.2 39) (end 50 39) (width 0.25) (layer F.Cu) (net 18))
 (segment (start 43.095 41.3) (end 43.095 39.905) (width 0.25) (layer F.Cu) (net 18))
 (segment (start 43.095 39.905) (end 45.1 37.9) (width 0.25) (layer F.Cu) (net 18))
 (segment (start 45.1 37.9) (end 47.1 37.9) (width 0.25) (layer F.Cu) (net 18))
 (segment (start 47.1 37.9) (end 48.2 39) (width 0.25) (layer F.Cu) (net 18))
 (segment (start 41.1 39) (end 39 39) (width 0.25) (layer F.Cu) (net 19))
 (segment (start 41.825 39.725) (end 41.1 39) (width 0.25) (layer F.Cu) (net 19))
 (segment (start 41.825 41.3) (end 41.825 39.725) (width 0.25) (layer F.Cu) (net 19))
 (segment (start 41.9 61) (end 39 61) (width 0.25) (layer F.Cu) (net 7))
 (segment (start 42.6 60.3) (end 41.9 61) (width 0.25) (layer F.Cu) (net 7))
 (segment (start 42.6 53.945) (end 42.6 60.3) (width 0.25) (layer F.Cu) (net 7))
 (segment (start 40.555 46.7) (end 40.555 47.855) (width 0.25) (layer F.Cu) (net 7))
 (segment (start 40.555 47.855) (end 40.9 48.2) (width 0.25) (layer F.Cu) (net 7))
 (segment (start 40.9 48.2) (end 40.9 52.245) (width 0.25) (layer F.Cu) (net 7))
 (segment (start 40.9 52.245) (end 42.6 53.945) (width 0.25) (layer F.Cu) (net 7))
 (segment (start 43.2 60.3) (end 43.9 61) (width 0.25) (layer F.Cu) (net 8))
 (segment (start 43.9 61) (end 50 61) (width 0.25) (layer F.Cu) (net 8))
 (segment (start 43.2 53.7) (end 43.2 60.3) (width 0.25) (layer F.Cu) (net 8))
 (segment (start 41.825 46.7) (end 41.825 47.7) (width 0.25) (layer F.Cu) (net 8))
 (segment (start 41.825 47.7) (end 41.350011 48.174989) (width 0.25) (layer F.Cu) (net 8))
 (segment (start 41.350011 48.174989) (end 41.350011 51.850011) (width 0.25) (layer F.Cu) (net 8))
 (segment (start 41.350011 51.850011) (end 43.2 53.7) (width 0.25) (layer F.Cu) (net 8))
 (segment (start 44.495 44.3) (end 43.095 45.7) (width 0.25) (layer F.Cu) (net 9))
 (segment (start 51.3 44.3) (end 44.495 44.3) (width 0.25) (layer F.Cu) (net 9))
 (segment (start 58.9 52.1) (end 58.4 52.6) (width 0.25) (layer F.Cu) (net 9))
 (segment (start 59.4 50) (end 58.9 50.5) (width 0.25) (layer F.Cu) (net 9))
 (segment (start 53.5 49) (end 52.3 47.8) (width 0.25) (layer F.Cu) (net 9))
 (segment (start 58.9 50.5) (end 58.9 52.1) (width 0.25) (layer F.Cu) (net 9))
 (segment (start 53.5 52.1) (end 53.5 49) (width 0.25) (layer F.Cu) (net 9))
 (segment (start 43.095 45.7) (end 43.095 46.7) (width 0.25) (layer F.Cu) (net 9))
 (segment (start 61 50) (end 59.4 50) (width 0.25) (layer F.Cu) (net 9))
 (segment (start 54 52.6) (end 53.5 52.1) (width 0.25) (layer F.Cu) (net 9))
 (segment (start 52.3 45.3) (end 51.3 44.3) (width 0.25) (layer F.Cu) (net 9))
 (segment (start 58.4 52.6) (end 54 52.6) (width 0.25) (layer F.Cu) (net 9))
 (segment (start 52.3 47.8) (end 52.3 45.3) (width 0.25) (layer F.Cu) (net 9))
 (segment (start 56.635 46.7) (end 56.635 45.675) (width 0.25) (layer F.Cu) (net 5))
 (via (at 56.65 45) (size 0.8) (drill 0.4) (layers F.Cu B.Cu) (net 5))
 (segment (start 56.635 45.015) (end 56.65 45) (width 0.25) (layer F.Cu) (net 5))
 (segment (start 56.635 46.7) (end 56.635 45.015) (width 0.25) (layer F.Cu) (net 5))
 (segment (start 56.65 45) (end 59.15 45) (width 0.25) (layer F.Cu) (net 5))
 (segment (start 59.75 45.6) (end 59.75 46.5) (width 0.25) (layer F.Cu) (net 5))
 (segment (start 59.15 45) (end 59.75 45.6) (width 0.25) (layer F.Cu) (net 5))
 (segment (start 48.175 42.725002) (end 48.15 42.750002) (width 0.25) (layer F.Cu) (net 5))
 (segment (start 48.175 41.3) (end 48.175 42.725002) (width 0.25) (layer F.Cu) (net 5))
 (via (at 48.15 42.750002) (size 0.8) (drill 0.4) (layers F.Cu B.Cu) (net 5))
 (segment (start 55.65 44) (end 56.65 45) (width 0.25) (layer B.Cu) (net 5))
 (segment (start 53.3 44) (end 55.65 44) (width 0.25) (layer B.Cu) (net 5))
 (segment (start 52.050002 42.750002) (end 53.3 44) (width 0.25) (layer B.Cu) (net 5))
 (segment (start 48.15 42.750002) (end 52.050002 42.750002) (width 0.25) (layer B.Cu) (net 5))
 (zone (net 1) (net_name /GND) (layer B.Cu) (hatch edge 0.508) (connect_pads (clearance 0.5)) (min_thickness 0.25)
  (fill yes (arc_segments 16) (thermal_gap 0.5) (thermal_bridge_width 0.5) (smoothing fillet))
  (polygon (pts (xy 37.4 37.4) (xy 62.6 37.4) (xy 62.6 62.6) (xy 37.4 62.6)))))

